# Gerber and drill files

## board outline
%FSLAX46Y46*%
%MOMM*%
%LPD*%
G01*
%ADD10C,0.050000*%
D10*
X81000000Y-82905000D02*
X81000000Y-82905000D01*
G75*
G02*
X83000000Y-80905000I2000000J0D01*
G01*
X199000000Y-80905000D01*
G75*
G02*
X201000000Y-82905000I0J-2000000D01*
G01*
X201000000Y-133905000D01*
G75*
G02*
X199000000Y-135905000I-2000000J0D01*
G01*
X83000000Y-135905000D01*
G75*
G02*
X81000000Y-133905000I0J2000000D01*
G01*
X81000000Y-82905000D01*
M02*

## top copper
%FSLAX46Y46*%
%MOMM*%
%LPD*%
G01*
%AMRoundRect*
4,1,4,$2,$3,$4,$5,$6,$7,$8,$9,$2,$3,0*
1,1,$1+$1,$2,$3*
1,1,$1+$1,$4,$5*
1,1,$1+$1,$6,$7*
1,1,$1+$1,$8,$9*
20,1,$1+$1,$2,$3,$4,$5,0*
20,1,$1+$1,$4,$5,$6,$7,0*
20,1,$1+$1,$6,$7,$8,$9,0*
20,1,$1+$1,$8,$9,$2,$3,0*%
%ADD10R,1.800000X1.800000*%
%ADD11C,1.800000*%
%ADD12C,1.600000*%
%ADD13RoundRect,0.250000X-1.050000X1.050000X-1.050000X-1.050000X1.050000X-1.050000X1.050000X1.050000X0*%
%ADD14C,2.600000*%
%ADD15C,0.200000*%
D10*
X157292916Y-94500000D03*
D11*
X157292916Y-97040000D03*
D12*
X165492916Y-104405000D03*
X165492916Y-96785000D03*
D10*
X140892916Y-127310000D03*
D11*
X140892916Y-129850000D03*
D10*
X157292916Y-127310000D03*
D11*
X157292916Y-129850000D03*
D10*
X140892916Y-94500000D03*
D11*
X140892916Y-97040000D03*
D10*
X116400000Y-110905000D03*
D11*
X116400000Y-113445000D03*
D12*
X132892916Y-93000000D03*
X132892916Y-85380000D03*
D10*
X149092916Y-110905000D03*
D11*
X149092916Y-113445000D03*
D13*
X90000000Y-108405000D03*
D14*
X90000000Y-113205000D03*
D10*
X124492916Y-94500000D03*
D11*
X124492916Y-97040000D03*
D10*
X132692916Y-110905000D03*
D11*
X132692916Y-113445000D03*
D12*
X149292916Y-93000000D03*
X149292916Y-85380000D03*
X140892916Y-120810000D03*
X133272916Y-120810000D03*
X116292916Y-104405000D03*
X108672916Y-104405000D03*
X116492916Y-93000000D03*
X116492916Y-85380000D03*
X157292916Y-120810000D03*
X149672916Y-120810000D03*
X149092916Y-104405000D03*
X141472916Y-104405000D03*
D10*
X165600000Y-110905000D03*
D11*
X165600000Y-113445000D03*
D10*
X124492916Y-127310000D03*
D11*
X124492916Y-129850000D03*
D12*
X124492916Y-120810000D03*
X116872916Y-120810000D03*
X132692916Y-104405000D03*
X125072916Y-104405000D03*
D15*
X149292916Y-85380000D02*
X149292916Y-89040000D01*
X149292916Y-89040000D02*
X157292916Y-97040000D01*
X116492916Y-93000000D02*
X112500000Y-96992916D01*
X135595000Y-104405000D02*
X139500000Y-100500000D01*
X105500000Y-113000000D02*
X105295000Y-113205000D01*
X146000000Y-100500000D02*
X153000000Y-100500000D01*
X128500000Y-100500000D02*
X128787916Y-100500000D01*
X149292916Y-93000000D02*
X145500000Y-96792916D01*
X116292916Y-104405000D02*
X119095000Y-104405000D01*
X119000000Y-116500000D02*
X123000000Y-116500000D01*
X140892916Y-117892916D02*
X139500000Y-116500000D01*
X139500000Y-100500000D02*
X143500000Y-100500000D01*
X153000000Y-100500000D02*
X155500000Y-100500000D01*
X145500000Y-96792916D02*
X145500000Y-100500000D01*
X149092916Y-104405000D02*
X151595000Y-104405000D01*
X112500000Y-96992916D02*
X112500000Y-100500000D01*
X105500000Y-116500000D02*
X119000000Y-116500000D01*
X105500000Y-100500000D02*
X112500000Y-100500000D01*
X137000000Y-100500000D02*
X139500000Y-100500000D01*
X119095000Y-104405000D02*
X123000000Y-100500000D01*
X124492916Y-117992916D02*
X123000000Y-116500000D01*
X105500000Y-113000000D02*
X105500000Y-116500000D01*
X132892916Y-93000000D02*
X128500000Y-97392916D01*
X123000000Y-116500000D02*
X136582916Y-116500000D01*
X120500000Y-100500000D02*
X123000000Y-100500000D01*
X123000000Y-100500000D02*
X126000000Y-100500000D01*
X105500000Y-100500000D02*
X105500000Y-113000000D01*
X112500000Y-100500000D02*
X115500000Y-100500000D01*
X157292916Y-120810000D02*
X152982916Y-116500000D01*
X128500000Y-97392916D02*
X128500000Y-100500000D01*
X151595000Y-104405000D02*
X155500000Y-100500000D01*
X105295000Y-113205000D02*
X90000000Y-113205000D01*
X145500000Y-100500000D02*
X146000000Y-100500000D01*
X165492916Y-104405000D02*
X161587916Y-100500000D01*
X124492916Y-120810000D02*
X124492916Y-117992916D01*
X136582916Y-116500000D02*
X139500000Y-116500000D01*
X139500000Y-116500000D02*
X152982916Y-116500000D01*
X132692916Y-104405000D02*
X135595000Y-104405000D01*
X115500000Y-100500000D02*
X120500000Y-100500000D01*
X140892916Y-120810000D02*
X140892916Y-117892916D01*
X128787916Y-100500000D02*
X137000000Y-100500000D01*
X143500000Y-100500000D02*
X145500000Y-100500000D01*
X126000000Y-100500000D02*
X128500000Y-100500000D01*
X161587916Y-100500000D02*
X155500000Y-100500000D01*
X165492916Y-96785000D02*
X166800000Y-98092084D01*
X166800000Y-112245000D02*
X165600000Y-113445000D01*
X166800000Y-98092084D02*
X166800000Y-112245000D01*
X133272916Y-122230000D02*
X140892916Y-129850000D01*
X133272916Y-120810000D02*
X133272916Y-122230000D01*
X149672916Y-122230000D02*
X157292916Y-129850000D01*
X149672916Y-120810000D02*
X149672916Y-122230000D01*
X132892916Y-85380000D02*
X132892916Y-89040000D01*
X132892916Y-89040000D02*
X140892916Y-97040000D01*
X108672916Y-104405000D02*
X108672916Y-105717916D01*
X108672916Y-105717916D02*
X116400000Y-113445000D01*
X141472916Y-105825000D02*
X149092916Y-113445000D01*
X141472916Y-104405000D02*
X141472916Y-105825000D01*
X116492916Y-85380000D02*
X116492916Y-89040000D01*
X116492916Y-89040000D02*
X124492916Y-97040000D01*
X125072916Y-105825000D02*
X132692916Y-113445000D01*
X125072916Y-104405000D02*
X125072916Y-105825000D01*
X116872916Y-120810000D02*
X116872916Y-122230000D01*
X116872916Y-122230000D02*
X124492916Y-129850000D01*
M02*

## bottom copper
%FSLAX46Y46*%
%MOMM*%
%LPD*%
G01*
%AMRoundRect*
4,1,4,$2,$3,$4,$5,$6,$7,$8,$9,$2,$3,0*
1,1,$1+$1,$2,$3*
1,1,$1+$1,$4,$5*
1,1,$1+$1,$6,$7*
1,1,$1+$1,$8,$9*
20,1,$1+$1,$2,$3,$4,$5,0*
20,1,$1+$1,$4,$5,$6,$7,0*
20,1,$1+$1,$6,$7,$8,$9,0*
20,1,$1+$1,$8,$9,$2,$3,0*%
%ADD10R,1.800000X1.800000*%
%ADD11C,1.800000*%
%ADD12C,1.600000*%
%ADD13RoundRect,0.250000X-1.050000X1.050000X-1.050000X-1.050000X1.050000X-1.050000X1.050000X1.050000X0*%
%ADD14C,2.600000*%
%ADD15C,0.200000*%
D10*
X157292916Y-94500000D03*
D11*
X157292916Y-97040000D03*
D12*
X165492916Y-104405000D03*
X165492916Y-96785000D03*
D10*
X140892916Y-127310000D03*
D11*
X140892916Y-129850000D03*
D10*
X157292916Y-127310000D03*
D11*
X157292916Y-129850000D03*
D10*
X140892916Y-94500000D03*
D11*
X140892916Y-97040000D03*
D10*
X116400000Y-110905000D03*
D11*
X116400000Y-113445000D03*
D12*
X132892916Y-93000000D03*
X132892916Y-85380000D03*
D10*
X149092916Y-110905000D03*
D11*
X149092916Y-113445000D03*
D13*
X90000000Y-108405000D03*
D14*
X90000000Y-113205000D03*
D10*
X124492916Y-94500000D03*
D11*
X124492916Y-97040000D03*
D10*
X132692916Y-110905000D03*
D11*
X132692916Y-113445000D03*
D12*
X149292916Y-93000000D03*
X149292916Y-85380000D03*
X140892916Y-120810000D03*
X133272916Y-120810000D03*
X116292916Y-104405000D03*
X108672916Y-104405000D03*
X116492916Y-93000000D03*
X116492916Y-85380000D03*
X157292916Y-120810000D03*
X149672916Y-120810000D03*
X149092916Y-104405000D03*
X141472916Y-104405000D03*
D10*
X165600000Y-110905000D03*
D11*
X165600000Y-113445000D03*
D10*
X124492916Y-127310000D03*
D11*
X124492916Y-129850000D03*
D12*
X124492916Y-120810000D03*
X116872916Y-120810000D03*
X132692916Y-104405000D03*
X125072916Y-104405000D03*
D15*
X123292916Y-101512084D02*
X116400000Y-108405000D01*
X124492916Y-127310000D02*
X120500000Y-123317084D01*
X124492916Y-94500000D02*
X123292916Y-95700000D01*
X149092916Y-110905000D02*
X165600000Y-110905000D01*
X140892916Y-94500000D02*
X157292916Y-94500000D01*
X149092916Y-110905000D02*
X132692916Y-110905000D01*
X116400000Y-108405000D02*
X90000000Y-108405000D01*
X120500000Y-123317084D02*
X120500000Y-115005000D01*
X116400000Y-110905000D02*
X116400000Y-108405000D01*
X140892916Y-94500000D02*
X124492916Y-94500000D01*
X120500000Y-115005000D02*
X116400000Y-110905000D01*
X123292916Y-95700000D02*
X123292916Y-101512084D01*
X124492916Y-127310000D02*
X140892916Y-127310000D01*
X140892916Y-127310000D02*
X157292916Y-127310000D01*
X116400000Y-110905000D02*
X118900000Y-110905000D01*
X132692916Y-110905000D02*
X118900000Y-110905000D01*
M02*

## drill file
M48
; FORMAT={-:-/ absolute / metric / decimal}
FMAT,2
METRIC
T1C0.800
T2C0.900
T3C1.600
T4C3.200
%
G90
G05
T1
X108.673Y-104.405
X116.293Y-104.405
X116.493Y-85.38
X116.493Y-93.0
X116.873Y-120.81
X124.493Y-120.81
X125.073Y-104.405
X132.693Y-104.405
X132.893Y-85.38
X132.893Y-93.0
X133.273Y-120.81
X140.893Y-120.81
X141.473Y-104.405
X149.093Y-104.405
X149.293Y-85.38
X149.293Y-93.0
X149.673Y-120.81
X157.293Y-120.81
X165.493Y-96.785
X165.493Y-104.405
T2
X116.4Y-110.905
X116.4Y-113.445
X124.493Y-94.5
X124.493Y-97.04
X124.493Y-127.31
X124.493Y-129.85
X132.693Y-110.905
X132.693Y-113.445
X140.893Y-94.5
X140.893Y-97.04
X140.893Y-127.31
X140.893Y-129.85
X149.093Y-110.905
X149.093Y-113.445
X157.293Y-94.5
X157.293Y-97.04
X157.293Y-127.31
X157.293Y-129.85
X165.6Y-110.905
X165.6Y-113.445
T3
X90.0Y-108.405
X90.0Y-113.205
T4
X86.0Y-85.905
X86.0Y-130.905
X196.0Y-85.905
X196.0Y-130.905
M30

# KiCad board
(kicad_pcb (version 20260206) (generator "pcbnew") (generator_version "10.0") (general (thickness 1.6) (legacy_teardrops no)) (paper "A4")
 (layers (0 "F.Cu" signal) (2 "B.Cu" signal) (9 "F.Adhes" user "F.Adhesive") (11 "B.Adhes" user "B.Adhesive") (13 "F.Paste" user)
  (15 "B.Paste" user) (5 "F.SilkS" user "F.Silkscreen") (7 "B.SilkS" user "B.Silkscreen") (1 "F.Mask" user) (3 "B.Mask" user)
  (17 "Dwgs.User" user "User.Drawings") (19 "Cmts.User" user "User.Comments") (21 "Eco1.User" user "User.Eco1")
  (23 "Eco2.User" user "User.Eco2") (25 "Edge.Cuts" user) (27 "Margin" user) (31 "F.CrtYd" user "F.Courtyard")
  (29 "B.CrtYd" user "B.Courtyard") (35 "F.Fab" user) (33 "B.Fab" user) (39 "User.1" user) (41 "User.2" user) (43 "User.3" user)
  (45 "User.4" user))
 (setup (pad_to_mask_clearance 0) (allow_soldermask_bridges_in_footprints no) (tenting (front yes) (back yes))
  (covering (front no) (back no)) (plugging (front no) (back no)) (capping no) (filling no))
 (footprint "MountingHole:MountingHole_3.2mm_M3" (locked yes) (layer "F.Cu") (at 196 85.905)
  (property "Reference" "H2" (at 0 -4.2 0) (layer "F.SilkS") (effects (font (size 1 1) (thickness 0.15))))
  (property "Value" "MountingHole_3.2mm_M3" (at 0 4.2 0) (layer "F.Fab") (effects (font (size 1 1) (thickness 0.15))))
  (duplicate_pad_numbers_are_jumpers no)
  (pad "" np_thru_hole circle (at 0 0) (size 3.2 3.2) (drill 3.2) (layers "*.Cu" "*.Mask")))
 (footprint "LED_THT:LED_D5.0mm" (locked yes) (layer "F.Cu") (at 157.292916 94.5 -90)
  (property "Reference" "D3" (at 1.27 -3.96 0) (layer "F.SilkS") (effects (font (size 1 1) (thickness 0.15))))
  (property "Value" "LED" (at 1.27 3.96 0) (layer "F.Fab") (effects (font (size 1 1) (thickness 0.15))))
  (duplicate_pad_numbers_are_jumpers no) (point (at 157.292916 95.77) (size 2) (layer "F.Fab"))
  (pad "1" thru_hole rect (at 0 0 270) (size 1.8 1.8) (drill 0.9) (layers "*.Cu" "*.Mask") (remove_unused_layers no) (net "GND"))
  (pad "2" thru_hole circle (at 2.54 0 270) (size 1.8 1.8) (drill 0.9) (layers "*.Cu" "*.Mask") (remove_unused_layers no) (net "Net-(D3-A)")))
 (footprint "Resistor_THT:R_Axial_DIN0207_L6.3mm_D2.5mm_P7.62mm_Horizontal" (layer "F.Cu") (at 165.492916 104.405 90)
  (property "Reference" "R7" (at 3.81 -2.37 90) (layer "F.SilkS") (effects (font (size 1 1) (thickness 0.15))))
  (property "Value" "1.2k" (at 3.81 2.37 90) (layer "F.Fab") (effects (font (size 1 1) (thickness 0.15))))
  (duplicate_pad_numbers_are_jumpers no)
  (pad "1" thru_hole circle (at 0 0 90) (size 1.6 1.6) (drill 0.8) (layers "*.Cu" "*.Mask") (remove_unused_layers no) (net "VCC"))
  (pad "2" thru_hole circle (at 7.62 0 90) (size 1.6 1.6) (drill 0.8) (layers "*.Cu" "*.Mask") (remove_unused_layers no) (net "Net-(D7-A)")))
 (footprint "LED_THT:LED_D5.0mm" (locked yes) (layer "F.Cu") (at 140.892916 127.31 -90)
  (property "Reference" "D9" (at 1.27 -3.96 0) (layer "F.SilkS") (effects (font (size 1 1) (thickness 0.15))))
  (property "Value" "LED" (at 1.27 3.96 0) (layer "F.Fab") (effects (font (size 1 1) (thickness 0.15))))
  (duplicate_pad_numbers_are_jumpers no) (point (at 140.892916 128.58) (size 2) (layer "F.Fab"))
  (pad "1" thru_hole rect (at 0 0 270) (size 1.8 1.8) (drill 0.9) (layers "*.Cu" "*.Mask") (remove_unused_layers no) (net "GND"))
  (pad "2" thru_hole circle (at 2.54 0 270) (size 1.8 1.8) (drill 0.9) (layers "*.Cu" "*.Mask") (remove_unused_layers no) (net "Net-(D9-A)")))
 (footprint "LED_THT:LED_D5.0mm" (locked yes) (layer "F.Cu") (at 157.292916 127.31 -90)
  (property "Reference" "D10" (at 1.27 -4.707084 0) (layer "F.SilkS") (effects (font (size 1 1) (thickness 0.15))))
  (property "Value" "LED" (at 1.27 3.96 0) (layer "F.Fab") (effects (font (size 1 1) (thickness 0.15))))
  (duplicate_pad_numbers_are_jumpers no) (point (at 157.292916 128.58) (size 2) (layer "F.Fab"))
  (pad "1" thru_hole rect (at 0 0 270) (size 1.8 1.8) (drill 0.9) (layers "*.Cu" "*.Mask") (remove_unused_layers no) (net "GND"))
  (pad "2" thru_hole circle (at 2.54 0 270) (size 1.8 1.8) (drill 0.9) (layers "*.Cu" "*.Mask") (remove_unused_layers no)
   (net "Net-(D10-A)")))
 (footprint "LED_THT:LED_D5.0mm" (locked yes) (layer "F.Cu") (at 140.892916 94.5 -90)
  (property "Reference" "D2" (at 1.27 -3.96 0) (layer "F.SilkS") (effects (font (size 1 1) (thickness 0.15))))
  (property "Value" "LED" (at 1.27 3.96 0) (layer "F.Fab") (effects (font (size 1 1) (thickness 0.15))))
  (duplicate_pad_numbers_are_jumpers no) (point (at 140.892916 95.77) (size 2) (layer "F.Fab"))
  (pad "1" thru_hole rect (at 0 0 270) (size 1.8 1.8) (drill 0.9) (layers "*.Cu" "*.Mask") (remove_unused_layers no) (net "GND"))
  (pad "2" thru_hole circle (at 2.54 0 270) (size 1.8 1.8) (drill 0.9) (layers "*.Cu" "*.Mask") (remove_unused_layers no) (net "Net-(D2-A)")))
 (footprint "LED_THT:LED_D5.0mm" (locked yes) (layer "F.Cu") (at 116.4 110.905 -90)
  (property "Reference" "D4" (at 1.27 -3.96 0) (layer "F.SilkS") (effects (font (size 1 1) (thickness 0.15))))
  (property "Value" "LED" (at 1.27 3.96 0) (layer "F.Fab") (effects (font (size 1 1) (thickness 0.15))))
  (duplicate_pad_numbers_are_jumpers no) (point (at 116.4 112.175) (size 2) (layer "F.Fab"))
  (pad "1" thru_hole rect (at 0 0 270) (size 1.8 1.8) (drill 0.9) (layers "*.Cu" "*.Mask") (remove_unused_layers no) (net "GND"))
  (pad "2" thru_hole circle (at 2.54 0 270) (size 1.8 1.8) (drill 0.9) (layers "*.Cu" "*.Mask") (remove_unused_layers no) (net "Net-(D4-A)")))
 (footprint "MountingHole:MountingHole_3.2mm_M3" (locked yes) (layer "F.Cu") (at 86 85.905)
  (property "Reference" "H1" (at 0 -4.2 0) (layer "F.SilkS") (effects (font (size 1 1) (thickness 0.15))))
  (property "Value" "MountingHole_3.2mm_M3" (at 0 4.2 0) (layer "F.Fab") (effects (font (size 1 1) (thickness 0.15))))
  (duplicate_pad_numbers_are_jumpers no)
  (pad "" np_thru_hole circle (at 0 0) (size 3.2 3.2) (drill 3.2) (layers "*.Cu" "*.Mask")))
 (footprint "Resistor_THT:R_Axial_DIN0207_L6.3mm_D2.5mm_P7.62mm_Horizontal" (layer "F.Cu") (at 132.892916 93 90)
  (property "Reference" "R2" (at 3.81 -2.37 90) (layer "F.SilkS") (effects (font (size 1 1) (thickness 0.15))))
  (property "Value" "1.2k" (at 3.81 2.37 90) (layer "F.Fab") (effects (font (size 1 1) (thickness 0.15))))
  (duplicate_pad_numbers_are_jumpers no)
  (pad "1" thru_hole circle (at 0 0 90) (size 1.6 1.6) (drill 0.8) (layers "*.Cu" "*.Mask") (remove_unused_layers no) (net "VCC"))
  (pad "2" thru_hole circle (at 7.62 0 90) (size 1.6 1.6) (drill 0.8) (layers "*.Cu" "*.Mask") (remove_unused_layers no) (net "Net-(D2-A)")))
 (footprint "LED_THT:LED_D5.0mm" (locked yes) (layer "F.Cu") (at 149.092916 110.905 -90)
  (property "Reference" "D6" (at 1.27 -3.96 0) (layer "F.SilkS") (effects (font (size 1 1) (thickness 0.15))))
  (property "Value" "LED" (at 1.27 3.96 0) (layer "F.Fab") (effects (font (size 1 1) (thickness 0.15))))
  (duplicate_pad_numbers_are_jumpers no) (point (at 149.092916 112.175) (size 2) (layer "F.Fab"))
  (pad "1" thru_hole rect (at 0 0 270) (size 1.8 1.8) (drill 0.9) (layers "*.Cu" "*.Mask") (remove_unused_layers no) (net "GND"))
  (pad "2" thru_hole circle (at 2.54 0 270) (size 1.8 1.8) (drill 0.9) (layers "*.Cu" "*.Mask") (remove_unused_layers no) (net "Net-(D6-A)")))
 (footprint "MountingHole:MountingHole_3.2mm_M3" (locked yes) (layer "F.Cu") (at 196 130.905)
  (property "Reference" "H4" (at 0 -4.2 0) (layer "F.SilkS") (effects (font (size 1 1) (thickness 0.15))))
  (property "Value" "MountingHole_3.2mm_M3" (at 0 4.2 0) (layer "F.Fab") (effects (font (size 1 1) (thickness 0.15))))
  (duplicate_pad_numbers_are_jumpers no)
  (pad "" np_thru_hole circle (at 0 0) (size 3.2 3.2) (drill 3.2) (layers "*.Cu" "*.Mask")))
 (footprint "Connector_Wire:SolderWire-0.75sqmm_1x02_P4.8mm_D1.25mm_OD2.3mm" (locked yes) (layer "F.Cu") (at 90 108.405 -90)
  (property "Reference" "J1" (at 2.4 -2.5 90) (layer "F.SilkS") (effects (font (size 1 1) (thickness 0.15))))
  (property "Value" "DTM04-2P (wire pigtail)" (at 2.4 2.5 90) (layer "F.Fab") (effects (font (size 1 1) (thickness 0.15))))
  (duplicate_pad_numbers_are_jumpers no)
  (pad "1" thru_hole roundrect (at 0 0 270) (size 2.6 2.6) (drill 1.6) (layers "*.Cu" "*.Mask") (remove_unused_layers no)
   (roundrect_rratio 0.096154) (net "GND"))
  (pad "2" thru_hole circle (at 4.8 0 270) (size 2.6 2.6) (drill 1.6) (layers "*.Cu" "*.Mask") (remove_unused_layers no) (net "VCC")))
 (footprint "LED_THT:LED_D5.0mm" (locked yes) (layer "F.Cu") (at 124.492916 94.5 -90)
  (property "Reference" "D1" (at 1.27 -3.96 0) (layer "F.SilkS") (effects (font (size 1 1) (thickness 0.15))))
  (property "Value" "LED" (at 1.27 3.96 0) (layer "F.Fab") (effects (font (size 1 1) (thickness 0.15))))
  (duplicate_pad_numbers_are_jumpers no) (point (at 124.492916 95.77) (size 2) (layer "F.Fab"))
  (pad "1" thru_hole rect (at 0 0 270) (size 1.8 1.8) (drill 0.9) (layers "*.Cu" "*.Mask") (remove_unused_layers no) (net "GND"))
  (pad "2" thru_hole circle (at 2.54 0 270) (size 1.8 1.8) (drill 0.9) (layers "*.Cu" "*.Mask") (remove_unused_layers no) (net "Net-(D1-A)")))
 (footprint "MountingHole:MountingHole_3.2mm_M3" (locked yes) (layer "F.Cu") (at 86 130.905)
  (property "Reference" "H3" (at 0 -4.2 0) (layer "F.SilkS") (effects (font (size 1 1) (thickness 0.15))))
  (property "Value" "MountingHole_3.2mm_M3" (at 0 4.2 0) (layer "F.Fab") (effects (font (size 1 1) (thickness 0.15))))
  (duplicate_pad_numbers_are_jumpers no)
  (pad "" np_thru_hole circle (at 0 0) (size 3.2 3.2) (drill 3.2) (layers "*.Cu" "*.Mask")))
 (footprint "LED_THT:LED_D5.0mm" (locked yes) (layer "F.Cu") (at 132.692916 110.905 -90)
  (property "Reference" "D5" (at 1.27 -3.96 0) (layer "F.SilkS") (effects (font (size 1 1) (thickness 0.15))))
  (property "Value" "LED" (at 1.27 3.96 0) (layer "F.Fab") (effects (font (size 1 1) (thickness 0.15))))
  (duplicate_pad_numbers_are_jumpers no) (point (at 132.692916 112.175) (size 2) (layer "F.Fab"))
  (pad "1" thru_hole rect (at 0 0 270) (size 1.8 1.8) (drill 0.9) (layers "*.Cu" "*.Mask") (remove_unused_layers no) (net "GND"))
  (pad "2" thru_hole circle (at 2.54 0 270) (size 1.8 1.8) (drill 0.9) (layers "*.Cu" "*.Mask") (remove_unused_layers no) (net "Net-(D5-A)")))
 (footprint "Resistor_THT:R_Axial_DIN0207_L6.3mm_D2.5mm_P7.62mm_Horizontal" (layer "F.Cu") (at 149.292916 93 90)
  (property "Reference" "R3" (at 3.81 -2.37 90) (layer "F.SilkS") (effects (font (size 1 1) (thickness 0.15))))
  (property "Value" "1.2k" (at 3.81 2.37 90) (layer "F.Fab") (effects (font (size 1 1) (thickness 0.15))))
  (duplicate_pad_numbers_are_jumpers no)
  (pad "1" thru_hole circle (at 0 0 90) (size 1.6 1.6) (drill 0.8) (layers "*.Cu" "*.Mask") (remove_unused_layers no) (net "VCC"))
  (pad "2" thru_hole circle (at 7.62 0 90) (size 1.6 1.6) (drill 0.8) (layers "*.Cu" "*.Mask") (remove_unused_layers no) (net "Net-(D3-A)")))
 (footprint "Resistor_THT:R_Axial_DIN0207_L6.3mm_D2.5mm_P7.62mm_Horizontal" (layer "F.Cu") (at 140.892916 120.81 180)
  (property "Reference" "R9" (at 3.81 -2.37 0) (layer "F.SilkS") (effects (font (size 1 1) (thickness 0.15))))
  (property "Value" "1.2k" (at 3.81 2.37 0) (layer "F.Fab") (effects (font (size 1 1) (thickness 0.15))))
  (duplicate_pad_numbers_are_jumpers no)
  (pad "1" thru_hole circle (at 0 0 180) (size 1.6 1.6) (drill 0.8) (layers "*.Cu" "*.Mask") (remove_unused_layers no) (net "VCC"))
  (pad "2" thru_hole circle (at 7.62 0 180) (size 1.6 1.6) (drill 0.8) (layers "*.Cu" "*.Mask") (remove_unused_layers no) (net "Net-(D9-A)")))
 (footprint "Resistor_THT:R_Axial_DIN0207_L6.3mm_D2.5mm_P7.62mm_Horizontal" (layer "F.Cu") (at 116.292916 104.405 180)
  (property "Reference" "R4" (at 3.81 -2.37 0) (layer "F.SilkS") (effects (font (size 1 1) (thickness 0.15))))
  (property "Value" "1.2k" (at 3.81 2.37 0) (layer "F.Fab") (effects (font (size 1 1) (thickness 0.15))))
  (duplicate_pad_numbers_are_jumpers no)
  (pad "1" thru_hole circle (at 0 0 180) (size 1.6 1.6) (drill 0.8) (layers "*.Cu" "*.Mask") (remove_unused_layers no) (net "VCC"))
  (pad "2" thru_hole circle (at 7.62 0 180) (size 1.6 1.6) (drill 0.8) (layers "*.Cu" "*.Mask") (remove_unused_layers no) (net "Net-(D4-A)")))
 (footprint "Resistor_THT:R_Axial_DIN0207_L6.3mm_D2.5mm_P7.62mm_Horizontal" (layer "F.Cu") (at 116.492916 93 90)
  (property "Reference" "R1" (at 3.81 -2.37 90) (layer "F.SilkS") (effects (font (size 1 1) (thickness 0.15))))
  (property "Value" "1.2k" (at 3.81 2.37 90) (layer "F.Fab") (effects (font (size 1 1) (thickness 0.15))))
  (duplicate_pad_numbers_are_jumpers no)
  (pad "1" thru_hole circle (at 0 0 90) (size 1.6 1.6) (drill 0.8) (layers "*.Cu" "*.Mask") (remove_unused_layers no) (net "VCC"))
  (pad "2" thru_hole circle (at 7.62 0 90) (size 1.6 1.6) (drill 0.8) (layers "*.Cu" "*.Mask") (remove_unused_layers no) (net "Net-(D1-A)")))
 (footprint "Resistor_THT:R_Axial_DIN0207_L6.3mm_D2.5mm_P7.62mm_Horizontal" (layer "F.Cu") (at 157.292916 120.81 180)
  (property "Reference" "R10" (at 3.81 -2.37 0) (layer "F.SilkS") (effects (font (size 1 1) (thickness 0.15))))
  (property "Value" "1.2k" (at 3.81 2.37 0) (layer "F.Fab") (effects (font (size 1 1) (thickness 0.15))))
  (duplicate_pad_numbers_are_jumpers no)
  (pad "1" thru_hole circle (at 0 0 180) (size 1.6 1.6) (drill 0.8) (layers "*.Cu" "*.Mask") (remove_unused_layers no) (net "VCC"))
  (pad "2" thru_hole circle (at 7.62 0 180) (size 1.6 1.6) (drill 0.8) (layers "*.Cu" "*.Mask") (remove_unused_layers no)
   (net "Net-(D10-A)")))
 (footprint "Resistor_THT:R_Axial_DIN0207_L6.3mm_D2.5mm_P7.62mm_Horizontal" (layer "F.Cu") (at 149.092916 104.405 180)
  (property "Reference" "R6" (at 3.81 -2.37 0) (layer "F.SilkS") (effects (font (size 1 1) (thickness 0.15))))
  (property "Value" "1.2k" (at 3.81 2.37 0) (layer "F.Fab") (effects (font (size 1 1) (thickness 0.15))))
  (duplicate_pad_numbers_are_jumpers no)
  (pad "1" thru_hole circle (at 0 0 180) (size 1.6 1.6) (drill 0.8) (layers "*.Cu" "*.Mask") (remove_unused_layers no) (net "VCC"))
  (pad "2" thru_hole circle (at 7.62 0 180) (size 1.6 1.6) (drill 0.8) (layers "*.Cu" "*.Mask") (remove_unused_layers no) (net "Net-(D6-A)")))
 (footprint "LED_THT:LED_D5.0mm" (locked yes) (layer "F.Cu") (at 165.6 110.905 -90)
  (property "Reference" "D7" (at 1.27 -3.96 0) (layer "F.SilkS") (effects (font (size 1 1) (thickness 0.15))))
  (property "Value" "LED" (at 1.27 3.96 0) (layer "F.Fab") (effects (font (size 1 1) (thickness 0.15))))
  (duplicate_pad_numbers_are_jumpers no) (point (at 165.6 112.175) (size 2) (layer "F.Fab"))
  (pad "1" thru_hole rect (at 0 0 270) (size 1.8 1.8) (drill 0.9) (layers "*.Cu" "*.Mask") (remove_unused_layers no) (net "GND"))
  (pad "2" thru_hole circle (at 2.54 0 270) (size 1.8 1.8) (drill 0.9) (layers "*.Cu" "*.Mask") (remove_unused_layers no) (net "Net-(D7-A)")))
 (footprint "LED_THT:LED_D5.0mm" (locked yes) (layer "F.Cu") (at 124.492916 127.31 -90)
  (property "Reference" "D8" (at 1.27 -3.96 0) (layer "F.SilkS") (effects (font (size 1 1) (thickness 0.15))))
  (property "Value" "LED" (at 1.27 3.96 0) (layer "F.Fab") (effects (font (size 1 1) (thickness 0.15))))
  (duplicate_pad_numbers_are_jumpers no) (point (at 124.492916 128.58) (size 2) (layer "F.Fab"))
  (pad "1" thru_hole rect (at 0 0 270) (size 1.8 1.8) (drill 0.9) (layers "*.Cu" "*.Mask") (remove_unused_layers no) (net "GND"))
  (pad "2" thru_hole circle (at 2.54 0 270) (size 1.8 1.8) (drill 0.9) (layers "*.Cu" "*.Mask") (remove_unused_layers no) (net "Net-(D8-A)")))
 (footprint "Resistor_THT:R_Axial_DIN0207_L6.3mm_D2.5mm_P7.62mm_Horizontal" (layer "F.Cu") (at 124.492916 120.81 180)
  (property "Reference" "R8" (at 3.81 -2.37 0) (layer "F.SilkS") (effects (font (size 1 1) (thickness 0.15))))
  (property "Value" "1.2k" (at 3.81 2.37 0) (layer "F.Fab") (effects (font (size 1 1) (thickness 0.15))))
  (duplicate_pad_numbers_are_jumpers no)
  (pad "1" thru_hole circle (at 0 0 180) (size 1.6 1.6) (drill 0.8) (layers "*.Cu" "*.Mask") (remove_unused_layers no) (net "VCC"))
  (pad "2" thru_hole circle (at 7.62 0 180) (size 1.6 1.6) (drill 0.8) (layers "*.Cu" "*.Mask") (remove_unused_layers no) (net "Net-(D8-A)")))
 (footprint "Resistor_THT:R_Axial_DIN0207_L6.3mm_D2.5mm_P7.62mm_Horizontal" (layer "F.Cu") (at 132.692916 104.405 180)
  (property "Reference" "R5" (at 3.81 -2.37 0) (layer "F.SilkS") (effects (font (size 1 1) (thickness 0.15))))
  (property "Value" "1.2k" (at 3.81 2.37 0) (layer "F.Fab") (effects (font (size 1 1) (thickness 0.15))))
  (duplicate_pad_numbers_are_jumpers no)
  (pad "1" thru_hole circle (at 0 0 180) (size 1.6 1.6) (drill 0.8) (layers "*.Cu" "*.Mask") (remove_unused_layers no) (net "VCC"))
  (pad "2" thru_hole circle (at 7.62 0 180) (size 1.6 1.6) (drill 0.8) (layers "*.Cu" "*.Mask") (remove_unused_layers no) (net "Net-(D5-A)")))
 (gr_rect (start 81 80.905) (end 201 135.905) (radius 2) (stroke (width 0.05) (type solid)) (fill no) (layer "Edge.Cuts"))
 (segment (start 123.292916 101.512084) (end 116.4 108.405) (width 0.2) (layer "B.Cu") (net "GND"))
 (segment (start 124.492916 127.31) (end 120.5 123.317084) (width 0.2) (layer "B.Cu") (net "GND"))
 (segment (start 124.492916 94.5) (end 123.292916 95.7) (width 0.2) (layer "B.Cu") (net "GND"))
 (segment (start 149.092916 110.905) (end 165.6 110.905) (width 0.2) (layer "B.Cu") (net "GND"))
 (segment (start 140.892916 94.5) (end 157.292916 94.5) (width 0.2) (layer "B.Cu") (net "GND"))
 (segment (start 149.092916 110.905) (end 132.692916 110.905) (width 0.2) (layer "B.Cu") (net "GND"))
 (segment (start 116.4 108.405) (end 90 108.405) (width 0.2) (layer "B.Cu") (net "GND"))
 (segment (start 120.5 123.317084) (end 120.5 115.005) (width 0.2) (layer "B.Cu") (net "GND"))
 (segment (start 116.4 110.905) (end 116.4 108.405) (width 0.2) (layer "B.Cu") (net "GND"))
 (segment (start 140.892916 94.5) (end 124.492916 94.5) (width 0.2) (layer "B.Cu") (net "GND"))
 (segment (start 120.5 115.005) (end 116.4 110.905) (width 0.2) (layer "B.Cu") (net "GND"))
 (segment (start 123.292916 95.7) (end 123.292916 101.512084) (width 0.2) (layer "B.Cu") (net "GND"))
 (segment (start 124.492916 127.31) (end 140.892916 127.31) (width 0.2) (layer "B.Cu") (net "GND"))
 (segment (start 140.892916 127.31) (end 157.292916 127.31) (width 0.2) (layer "B.Cu") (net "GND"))
 (segment (start 116.4 110.905) (end 118.9 110.905) (width 0.2) (layer "B.Cu") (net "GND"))
 (segment (start 132.692916 110.905) (end 118.9 110.905) (width 0.2) (layer "B.Cu") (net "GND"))
 (segment (start 149.292916 85.38) (end 149.292916 89.04) (width 0.2) (layer "F.Cu") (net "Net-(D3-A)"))
 (segment (start 149.292916 89.04) (end 157.292916 97.04) (width 0.2) (layer "F.Cu") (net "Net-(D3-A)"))
 (segment (start 116.492916 93) (end 112.5 96.992916) (width 0.2) (layer "F.Cu") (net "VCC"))
 (segment (start 135.595 104.405) (end 139.5 100.5) (width 0.2) (layer "F.Cu") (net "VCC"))
 (segment (start 105.5 113) (end 105.295 113.205) (width 0.2) (layer "F.Cu") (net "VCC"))
 (segment (start 146 100.5) (end 153 100.5) (width 0.2) (layer "F.Cu") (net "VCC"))
 (segment (start 128.5 100.5) (end 128.787916 100.5) (width 0.2) (layer "F.Cu") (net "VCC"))
 (segment (start 149.292916 93) (end 145.5 96.792916) (width 0.2) (layer "F.Cu") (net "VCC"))
 (segment (start 116.292916 104.405) (end 119.095 104.405) (width 0.2) (layer "F.Cu") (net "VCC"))
 (segment (start 119 116.5) (end 123 116.5) (width 0.2) (layer "F.Cu") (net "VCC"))
 (segment (start 140.892916 117.892916) (end 139.5 116.5) (width 0.2) (layer "F.Cu") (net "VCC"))
 (segment (start 139.5 100.5) (end 143.5 100.5) (width 0.2) (layer "F.Cu") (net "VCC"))
 (segment (start 153 100.5) (end 155.5 100.5) (width 0.2) (layer "F.Cu") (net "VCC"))
 (segment (start 145.5 96.792916) (end 145.5 100.5) (width 0.2) (layer "F.Cu") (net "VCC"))
 (segment (start 149.092916 104.405) (end 151.595 104.405) (width 0.2) (layer "F.Cu") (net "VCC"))
 (segment (start 112.5 96.992916) (end 112.5 100.5) (width 0.2) (layer "F.Cu") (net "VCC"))
 (segment (start 105.5 116.5) (end 119 116.5) (width 0.2) (layer "F.Cu") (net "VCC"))
 (segment (start 105.5 100.5) (end 112.5 100.5) (width 0.2) (layer "F.Cu") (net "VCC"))
 (segment (start 137 100.5) (end 139.5 100.5) (width 0.2) (layer "F.Cu") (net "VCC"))
 (segment (start 119.095 104.405) (end 123 100.5) (width 0.2) (layer "F.Cu") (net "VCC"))
 (segment (start 124.492916 117.992916) (end 123 116.5) (width 0.2) (layer "F.Cu") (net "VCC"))
 (segment (start 105.5 113) (end 105.5 116.5) (width 0.2) (layer "F.Cu") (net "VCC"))
 (segment (start 132.892916 93) (end 128.5 97.392916) (width 0.2) (layer "F.Cu") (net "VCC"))
 (segment (start 123 116.5) (end 136.582916 116.5) (width 0.2) (layer "F.Cu") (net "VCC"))
 (segment (start 120.5 100.5) (end 123 100.5) (width 0.2) (layer "F.Cu") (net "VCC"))
 (segment (start 123 100.5) (end 126 100.5) (width 0.2) (layer "F.Cu") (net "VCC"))
 (segment (start 105.5 100.5) (end 105.5 113) (width 0.2) (layer "F.Cu") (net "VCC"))
 (segment (start 112.5 100.5) (end 115.5 100.5) (width 0.2) (layer "F.Cu") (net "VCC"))
 (segment (start 157.292916 120.81) (end 152.982916 116.5) (width 0.2) (layer "F.Cu") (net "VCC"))
 (segment (start 128.5 97.392916) (end 128.5 100.5) (width 0.2) (layer "F.Cu") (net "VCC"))
 (segment (start 151.595 104.405) (end 155.5 100.5) (width 0.2) (layer "F.Cu") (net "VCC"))
 (segment (start 105.295 113.205) (end 90 113.205) (width 0.2) (layer "F.Cu") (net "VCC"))
 (segment (start 145.5 100.5) (end 146 100.5) (width 0.2) (layer "F.Cu") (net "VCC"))
 (segment (start 165.492916 104.405) (end 161.587916 100.5) (width 0.2) (layer "F.Cu") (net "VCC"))
 (segment (start 124.492916 120.81) (end 124.492916 117.992916) (width 0.2) (layer "F.Cu") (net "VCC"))
 (segment (start 136.582916 116.5) (end 139.5 116.5) (width 0.2) (layer "F.Cu") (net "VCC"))
 (segment (start 139.5 116.5) (end 152.982916 116.5) (width 0.2) (layer "F.Cu") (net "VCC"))
 (segment (start 132.692916 104.405) (end 135.595 104.405) (width 0.2) (layer "F.Cu") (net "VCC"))
 (segment (start 115.5 100.5) (end 120.5 100.5) (width 0.2) (layer "F.Cu") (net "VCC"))
 (segment (start 140.892916 120.81) (end 140.892916 117.892916) (width 0.2) (layer "F.Cu") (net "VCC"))
 (segment (start 128.787916 100.5) (end 137 100.5) (width 0.2) (layer "F.Cu") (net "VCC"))
 (segment (start 143.5 100.5) (end 145.5 100.5) (width 0.2) (layer "F.Cu") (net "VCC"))
 (segment (start 126 100.5) (end 128.5 100.5) (width 0.2) (layer "F.Cu") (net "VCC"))
 (segment (start 161.587916 100.5) (end 155.5 100.5) (width 0.2) (layer "F.Cu") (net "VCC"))
 (segment (start 165.492916 96.785) (end 166.8 98.092084) (width 0.2) (layer "F.Cu") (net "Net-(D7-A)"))
 (segment (start 166.8 112.245) (end 165.6 113.445) (width 0.2) (layer "F.Cu") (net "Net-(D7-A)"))
 (segment (start 166.8 98.092084) (end 166.8 112.245) (width 0.2) (layer "F.Cu") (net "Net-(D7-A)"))
 (segment (start 133.272916 122.23) (end 140.892916 129.85) (width 0.2) (layer "F.Cu") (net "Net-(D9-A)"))
 (segment (start 133.272916 120.81) (end 133.272916 122.23) (width 0.2) (layer "F.Cu") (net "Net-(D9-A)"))
 (segment (start 149.672916 122.23) (end 157.292916 129.85) (width 0.2) (layer "F.Cu") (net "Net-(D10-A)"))
 (segment (start 149.672916 120.81) (end 149.672916 122.23) (width 0.2) (layer "F.Cu") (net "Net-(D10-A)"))
 (segment (start 132.892916 85.38) (end 132.892916 89.04) (width 0.2) (layer "F.Cu") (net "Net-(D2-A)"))
 (segment (start 132.892916 89.04) (end 140.892916 97.04) (width 0.2) (layer "F.Cu") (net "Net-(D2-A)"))
 (segment (start 108.672916 104.405) (end 108.672916 105.717916) (width 0.2) (layer "F.Cu") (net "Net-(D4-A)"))
 (segment (start 108.672916 105.717916) (end 116.4 113.445) (width 0.2) (layer "F.Cu") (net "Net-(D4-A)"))
 (segment (start 141.472916 105.825) (end 149.092916 113.445) (width 0.2) (layer "F.Cu") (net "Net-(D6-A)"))
 (segment (start 141.472916 104.405) (end 141.472916 105.825) (width 0.2) (layer "F.Cu") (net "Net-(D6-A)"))
 (segment (start 116.492916 85.38) (end 116.492916 89.04) (width 0.2) (layer "F.Cu") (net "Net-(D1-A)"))
 (segment (start 116.492916 89.04) (end 124.492916 97.04) (width 0.2) (layer "F.Cu") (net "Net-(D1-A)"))
 (segment (start 125.072916 105.825) (end 132.692916 113.445) (width 0.2) (layer "F.Cu") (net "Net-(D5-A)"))
 (segment (start 125.072916 104.405) (end 125.072916 105.825) (width 0.2) (layer "F.Cu") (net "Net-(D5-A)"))
 (segment (start 116.872916 120.81) (end 116.872916 122.23) (width 0.2) (layer "F.Cu") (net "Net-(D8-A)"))
 (segment (start 116.872916 122.23) (end 124.492916 129.85) (width 0.2) (layer "F.Cu") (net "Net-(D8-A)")))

